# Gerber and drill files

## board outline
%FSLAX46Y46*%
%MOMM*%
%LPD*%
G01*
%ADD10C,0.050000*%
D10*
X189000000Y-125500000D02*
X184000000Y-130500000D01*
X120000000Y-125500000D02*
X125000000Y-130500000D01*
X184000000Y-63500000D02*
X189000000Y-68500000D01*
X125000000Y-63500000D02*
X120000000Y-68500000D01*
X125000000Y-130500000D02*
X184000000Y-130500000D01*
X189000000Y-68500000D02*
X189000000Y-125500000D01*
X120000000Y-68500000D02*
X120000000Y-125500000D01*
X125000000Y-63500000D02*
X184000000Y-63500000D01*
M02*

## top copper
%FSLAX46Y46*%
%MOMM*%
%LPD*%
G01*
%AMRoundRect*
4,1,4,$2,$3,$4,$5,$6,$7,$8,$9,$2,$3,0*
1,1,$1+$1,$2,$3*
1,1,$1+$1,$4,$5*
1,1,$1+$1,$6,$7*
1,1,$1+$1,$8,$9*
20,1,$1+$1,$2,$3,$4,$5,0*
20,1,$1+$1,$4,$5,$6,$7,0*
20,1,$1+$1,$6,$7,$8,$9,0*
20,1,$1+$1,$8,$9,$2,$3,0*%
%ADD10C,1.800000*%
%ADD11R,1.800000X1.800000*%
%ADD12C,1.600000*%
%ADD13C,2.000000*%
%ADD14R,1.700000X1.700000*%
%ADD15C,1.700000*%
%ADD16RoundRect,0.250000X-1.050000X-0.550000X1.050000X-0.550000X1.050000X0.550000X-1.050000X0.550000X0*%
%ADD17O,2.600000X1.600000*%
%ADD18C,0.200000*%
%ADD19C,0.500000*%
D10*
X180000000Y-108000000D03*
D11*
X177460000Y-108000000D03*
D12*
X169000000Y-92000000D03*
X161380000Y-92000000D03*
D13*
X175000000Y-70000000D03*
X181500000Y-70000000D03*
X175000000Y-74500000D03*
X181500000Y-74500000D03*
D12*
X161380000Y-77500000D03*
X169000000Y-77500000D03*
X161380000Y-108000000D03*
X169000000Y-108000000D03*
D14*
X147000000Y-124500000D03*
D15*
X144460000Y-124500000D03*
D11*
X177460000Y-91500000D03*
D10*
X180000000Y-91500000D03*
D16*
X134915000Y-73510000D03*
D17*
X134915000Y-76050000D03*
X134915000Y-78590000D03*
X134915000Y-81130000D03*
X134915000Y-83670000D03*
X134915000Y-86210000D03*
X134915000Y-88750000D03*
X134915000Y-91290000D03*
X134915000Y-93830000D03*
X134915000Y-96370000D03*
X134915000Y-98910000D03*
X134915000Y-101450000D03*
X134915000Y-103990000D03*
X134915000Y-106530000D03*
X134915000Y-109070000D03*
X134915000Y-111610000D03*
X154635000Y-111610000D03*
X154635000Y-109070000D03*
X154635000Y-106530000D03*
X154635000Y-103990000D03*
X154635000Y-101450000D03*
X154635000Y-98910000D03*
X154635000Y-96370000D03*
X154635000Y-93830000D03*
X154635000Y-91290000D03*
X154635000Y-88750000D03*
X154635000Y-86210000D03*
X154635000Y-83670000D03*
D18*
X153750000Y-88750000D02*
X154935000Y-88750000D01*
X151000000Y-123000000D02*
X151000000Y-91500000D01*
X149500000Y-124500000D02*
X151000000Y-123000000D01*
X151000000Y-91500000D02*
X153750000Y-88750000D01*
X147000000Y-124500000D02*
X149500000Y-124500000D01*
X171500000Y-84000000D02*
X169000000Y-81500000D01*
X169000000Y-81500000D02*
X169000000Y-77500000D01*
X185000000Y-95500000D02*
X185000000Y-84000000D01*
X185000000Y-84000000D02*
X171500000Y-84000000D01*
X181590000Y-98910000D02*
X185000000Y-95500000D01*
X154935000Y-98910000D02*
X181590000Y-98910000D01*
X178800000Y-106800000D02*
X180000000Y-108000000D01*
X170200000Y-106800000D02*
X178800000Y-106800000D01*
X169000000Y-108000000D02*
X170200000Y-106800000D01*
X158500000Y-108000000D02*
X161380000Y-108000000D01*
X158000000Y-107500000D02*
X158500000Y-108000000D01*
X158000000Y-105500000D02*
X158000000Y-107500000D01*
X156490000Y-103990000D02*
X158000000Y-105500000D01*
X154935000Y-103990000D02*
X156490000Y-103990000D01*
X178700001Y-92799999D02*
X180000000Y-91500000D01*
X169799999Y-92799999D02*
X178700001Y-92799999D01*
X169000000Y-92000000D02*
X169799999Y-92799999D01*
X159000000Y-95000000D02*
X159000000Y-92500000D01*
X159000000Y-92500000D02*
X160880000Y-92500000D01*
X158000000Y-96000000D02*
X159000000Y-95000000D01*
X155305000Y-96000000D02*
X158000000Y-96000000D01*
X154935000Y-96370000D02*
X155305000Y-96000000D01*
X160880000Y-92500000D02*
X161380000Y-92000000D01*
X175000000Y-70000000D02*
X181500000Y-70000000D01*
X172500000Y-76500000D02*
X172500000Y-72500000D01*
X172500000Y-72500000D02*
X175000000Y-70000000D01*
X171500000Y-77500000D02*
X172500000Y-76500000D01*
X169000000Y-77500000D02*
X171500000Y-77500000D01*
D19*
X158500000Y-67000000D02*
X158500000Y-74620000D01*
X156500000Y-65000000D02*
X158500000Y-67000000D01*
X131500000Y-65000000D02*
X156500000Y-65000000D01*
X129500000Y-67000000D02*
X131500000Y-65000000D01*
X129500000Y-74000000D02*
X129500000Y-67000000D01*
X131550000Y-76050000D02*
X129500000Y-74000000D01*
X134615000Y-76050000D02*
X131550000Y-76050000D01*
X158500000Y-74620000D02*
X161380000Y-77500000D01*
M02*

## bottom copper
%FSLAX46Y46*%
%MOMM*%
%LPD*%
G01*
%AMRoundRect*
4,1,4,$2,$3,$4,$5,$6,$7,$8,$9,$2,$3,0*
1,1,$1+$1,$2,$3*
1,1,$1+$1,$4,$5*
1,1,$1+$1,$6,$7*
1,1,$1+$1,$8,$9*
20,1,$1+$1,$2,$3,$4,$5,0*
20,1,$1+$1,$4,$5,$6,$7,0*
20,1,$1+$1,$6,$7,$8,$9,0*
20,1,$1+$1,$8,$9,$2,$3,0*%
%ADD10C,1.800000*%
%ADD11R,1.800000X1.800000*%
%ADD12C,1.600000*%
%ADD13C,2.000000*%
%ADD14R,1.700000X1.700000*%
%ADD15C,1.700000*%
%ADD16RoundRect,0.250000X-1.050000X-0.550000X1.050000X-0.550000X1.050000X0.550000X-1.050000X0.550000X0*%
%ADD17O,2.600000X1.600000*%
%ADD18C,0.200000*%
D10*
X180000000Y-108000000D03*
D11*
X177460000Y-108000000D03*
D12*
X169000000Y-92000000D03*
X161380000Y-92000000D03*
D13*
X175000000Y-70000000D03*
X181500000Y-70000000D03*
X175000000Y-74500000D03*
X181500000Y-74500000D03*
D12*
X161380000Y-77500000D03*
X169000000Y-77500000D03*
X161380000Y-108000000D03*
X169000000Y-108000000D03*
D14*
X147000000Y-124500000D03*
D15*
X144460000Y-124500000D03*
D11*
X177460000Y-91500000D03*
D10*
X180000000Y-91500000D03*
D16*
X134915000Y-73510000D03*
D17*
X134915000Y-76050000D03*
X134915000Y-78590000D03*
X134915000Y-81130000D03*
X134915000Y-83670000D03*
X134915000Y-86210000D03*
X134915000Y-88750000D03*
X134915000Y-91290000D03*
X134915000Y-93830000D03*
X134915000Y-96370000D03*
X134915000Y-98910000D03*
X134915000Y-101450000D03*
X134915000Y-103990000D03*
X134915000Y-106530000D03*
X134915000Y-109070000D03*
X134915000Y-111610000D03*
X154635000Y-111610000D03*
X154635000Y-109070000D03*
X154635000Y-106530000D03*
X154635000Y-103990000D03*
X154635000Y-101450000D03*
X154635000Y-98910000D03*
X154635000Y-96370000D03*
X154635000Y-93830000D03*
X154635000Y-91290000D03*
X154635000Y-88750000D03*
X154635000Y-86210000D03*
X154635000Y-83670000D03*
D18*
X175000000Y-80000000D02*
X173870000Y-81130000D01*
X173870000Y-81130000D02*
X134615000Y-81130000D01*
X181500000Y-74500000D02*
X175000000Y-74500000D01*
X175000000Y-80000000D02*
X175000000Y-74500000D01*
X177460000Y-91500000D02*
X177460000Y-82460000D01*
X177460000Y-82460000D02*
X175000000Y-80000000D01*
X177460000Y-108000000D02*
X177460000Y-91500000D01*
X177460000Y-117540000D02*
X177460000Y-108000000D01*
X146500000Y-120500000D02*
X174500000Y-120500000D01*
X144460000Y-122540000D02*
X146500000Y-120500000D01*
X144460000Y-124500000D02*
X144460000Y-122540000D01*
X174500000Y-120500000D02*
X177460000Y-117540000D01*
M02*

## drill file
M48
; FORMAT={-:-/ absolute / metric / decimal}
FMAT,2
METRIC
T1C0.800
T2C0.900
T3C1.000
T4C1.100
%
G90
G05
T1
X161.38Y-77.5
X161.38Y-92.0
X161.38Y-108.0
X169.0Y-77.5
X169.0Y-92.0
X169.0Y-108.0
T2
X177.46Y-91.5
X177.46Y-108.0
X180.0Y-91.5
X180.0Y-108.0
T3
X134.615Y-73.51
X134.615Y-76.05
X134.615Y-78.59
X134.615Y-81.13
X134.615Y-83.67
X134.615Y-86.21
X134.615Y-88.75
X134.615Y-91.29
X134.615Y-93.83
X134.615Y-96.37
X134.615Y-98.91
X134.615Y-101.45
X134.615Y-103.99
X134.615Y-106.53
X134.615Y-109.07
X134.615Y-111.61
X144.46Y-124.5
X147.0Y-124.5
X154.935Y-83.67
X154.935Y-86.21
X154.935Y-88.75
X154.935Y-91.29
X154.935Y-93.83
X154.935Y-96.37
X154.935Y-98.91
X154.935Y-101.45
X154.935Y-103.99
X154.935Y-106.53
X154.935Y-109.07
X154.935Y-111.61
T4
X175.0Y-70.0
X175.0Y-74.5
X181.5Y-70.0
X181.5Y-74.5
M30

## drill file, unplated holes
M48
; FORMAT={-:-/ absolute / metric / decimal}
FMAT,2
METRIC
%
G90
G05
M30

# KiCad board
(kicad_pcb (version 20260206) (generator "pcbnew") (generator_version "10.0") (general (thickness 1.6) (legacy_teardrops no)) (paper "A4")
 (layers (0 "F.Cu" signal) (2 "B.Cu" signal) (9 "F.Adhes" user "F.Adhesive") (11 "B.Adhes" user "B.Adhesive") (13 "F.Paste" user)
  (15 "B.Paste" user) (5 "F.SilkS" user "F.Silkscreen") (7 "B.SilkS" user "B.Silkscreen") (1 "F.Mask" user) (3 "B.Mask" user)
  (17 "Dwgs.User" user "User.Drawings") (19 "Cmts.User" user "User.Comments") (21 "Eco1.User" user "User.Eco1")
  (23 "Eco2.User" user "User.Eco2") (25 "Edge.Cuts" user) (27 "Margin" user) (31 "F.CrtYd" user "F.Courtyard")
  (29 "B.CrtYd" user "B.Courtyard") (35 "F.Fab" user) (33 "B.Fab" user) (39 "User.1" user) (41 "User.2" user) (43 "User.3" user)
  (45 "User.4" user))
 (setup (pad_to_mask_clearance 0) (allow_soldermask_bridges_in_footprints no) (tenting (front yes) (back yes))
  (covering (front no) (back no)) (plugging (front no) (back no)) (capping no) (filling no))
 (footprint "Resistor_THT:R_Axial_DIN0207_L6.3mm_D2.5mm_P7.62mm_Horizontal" (layer "F.Cu") (at 161.38 108)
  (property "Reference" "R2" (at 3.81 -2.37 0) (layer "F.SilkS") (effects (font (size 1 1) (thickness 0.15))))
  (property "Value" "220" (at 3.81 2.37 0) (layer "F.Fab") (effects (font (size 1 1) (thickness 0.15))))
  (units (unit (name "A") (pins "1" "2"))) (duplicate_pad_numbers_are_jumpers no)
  (pad "1" thru_hole circle (at 0 0) (size 1.6 1.6) (drill 0.8) (layers "*.Cu" "*.Mask") (remove_unused_layers no)
   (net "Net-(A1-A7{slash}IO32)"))
  (pad "2" thru_hole circle (at 7.62 0) (size 1.6 1.6) (drill 0.8) (layers "*.Cu" "*.Mask") (remove_unused_layers no) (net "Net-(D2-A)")))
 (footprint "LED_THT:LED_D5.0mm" (layer "F.Cu") (at 177.46 91.5)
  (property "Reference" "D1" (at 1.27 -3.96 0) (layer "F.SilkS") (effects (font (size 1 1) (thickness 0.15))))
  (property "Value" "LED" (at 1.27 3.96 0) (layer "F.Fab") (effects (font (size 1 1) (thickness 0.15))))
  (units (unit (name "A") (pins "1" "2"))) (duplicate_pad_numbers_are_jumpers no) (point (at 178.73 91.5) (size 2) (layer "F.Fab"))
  (pad "1" thru_hole rect (at 0 0) (size 1.8 1.8) (drill 0.9) (layers "*.Cu" "*.Mask") (remove_unused_layers no) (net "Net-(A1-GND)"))
  (pad "2" thru_hole circle (at 2.54 0) (size 1.8 1.8) (drill 0.9) (layers "*.Cu" "*.Mask") (remove_unused_layers no) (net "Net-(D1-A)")))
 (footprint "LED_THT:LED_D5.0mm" (layer "F.Cu") (at 177.46 108)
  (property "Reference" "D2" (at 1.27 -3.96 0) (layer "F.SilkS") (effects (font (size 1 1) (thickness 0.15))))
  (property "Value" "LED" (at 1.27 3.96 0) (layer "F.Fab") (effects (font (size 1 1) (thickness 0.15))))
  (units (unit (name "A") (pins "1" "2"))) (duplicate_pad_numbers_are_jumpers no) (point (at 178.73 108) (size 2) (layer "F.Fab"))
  (pad "1" thru_hole rect (at 0 0) (size 1.8 1.8) (drill 0.9) (layers "*.Cu" "*.Mask") (remove_unused_layers no) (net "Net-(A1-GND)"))
  (pad "2" thru_hole circle (at 2.54 0) (size 1.8 1.8) (drill 0.9) (layers "*.Cu" "*.Mask") (remove_unused_layers no) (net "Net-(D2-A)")))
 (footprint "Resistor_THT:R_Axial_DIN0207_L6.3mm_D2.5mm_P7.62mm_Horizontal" (layer "F.Cu") (at 161.38 92)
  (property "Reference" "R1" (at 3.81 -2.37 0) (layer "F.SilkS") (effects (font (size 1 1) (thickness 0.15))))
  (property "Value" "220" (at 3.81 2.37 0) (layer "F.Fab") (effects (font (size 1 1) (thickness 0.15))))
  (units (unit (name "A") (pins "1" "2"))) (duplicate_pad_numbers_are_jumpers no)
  (pad "1" thru_hole circle (at 0 0) (size 1.6 1.6) (drill 0.8) (layers "*.Cu" "*.Mask") (remove_unused_layers no)
   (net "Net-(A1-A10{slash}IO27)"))
  (pad "2" thru_hole circle (at 7.62 0) (size 1.6 1.6) (drill 0.8) (layers "*.Cu" "*.Mask") (remove_unused_layers no) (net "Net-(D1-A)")))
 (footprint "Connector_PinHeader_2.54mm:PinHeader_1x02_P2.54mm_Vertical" (layer "F.Cu") (at 147 124.5 -90)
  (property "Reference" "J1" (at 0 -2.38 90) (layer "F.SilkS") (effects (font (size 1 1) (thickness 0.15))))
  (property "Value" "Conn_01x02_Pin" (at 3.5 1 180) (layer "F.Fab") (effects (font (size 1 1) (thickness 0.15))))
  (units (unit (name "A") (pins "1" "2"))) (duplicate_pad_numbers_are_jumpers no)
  (pad "1" thru_hole rect (at 0 0 270) (size 1.7 1.7) (drill 1) (layers "*.Cu" "*.Mask") (remove_unused_layers no) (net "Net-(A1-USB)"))
  (pad "2" thru_hole circle (at 0 2.54 270) (size 1.7 1.7) (drill 1) (layers "*.Cu" "*.Mask") (remove_unused_layers no) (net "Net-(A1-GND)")))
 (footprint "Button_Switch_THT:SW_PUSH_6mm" (layer "F.Cu") (at 175 70)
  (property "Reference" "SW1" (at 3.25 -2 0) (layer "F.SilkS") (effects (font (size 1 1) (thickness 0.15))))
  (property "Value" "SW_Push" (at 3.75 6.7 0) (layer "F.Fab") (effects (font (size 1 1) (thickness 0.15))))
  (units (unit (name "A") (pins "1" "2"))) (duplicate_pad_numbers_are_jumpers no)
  (pad "1" thru_hole circle (at 0 0 90) (size 2 2) (drill 1.1) (layers "*.Cu" "*.Mask") (remove_unused_layers no)
   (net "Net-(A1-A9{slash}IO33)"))
  (pad "1" thru_hole circle (at 6.5 0 90) (size 2 2) (drill 1.1) (layers "*.Cu" "*.Mask") (remove_unused_layers no)
   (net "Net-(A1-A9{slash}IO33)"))
  (pad "2" thru_hole circle (at 0 4.5 90) (size 2 2) (drill 1.1) (layers "*.Cu" "*.Mask") (remove_unused_layers no) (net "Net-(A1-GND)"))
  (pad "2" thru_hole circle (at 6.5 4.5 90) (size 2 2) (drill 1.1) (layers "*.Cu" "*.Mask") (remove_unused_layers no) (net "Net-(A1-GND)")))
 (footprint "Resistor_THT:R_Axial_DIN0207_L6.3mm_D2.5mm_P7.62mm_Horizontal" (layer "F.Cu") (at 161.38 77.5)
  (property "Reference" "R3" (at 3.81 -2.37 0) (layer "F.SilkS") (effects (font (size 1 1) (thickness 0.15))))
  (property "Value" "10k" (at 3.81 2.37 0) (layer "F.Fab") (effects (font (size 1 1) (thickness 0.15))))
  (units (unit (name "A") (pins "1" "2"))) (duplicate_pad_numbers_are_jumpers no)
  (pad "1" thru_hole circle (at 0 0) (size 1.6 1.6) (drill 0.8) (layers "*.Cu" "*.Mask") (remove_unused_layers no) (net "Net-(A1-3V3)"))
  (pad "2" thru_hole circle (at 7.62 0) (size 1.6 1.6) (drill 0.8) (layers "*.Cu" "*.Mask") (remove_unused_layers no)
   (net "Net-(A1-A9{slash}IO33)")))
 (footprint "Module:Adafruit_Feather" (layer "F.Cu") (at 134.615 73.51)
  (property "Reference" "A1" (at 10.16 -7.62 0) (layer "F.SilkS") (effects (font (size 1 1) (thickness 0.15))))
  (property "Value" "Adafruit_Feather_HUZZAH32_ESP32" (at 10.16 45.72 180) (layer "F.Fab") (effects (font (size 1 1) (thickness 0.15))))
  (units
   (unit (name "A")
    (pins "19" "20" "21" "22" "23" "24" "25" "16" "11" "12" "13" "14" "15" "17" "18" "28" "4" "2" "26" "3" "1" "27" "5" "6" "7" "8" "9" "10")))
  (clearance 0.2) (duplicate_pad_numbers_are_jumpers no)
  (pad "1" thru_hole roundrect (at 0 0) (size 2.6 1.6) (drill 1 (offset 0.3 0)) (layers "*.Cu" "*.Mask") (remove_unused_layers no)
   (roundrect_rratio 0.15625) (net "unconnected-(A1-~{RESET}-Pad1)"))
  (pad "2" thru_hole oval (at 0 2.54) (size 2.6 1.6) (drill 1 (offset 0.3 0)) (layers "*.Cu" "*.Mask") (remove_unused_layers no)
   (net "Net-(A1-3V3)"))
  (pad "3" thru_hole oval (at 0 5.08) (size 2.6 1.6) (drill 1 (offset 0.3 0)) (layers "*.Cu" "*.Mask") (remove_unused_layers no)
   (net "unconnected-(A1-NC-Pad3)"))
  (pad "4" thru_hole oval (at 0 7.62) (size 2.6 1.6) (drill 1 (offset 0.3 0)) (layers "*.Cu" "*.Mask") (remove_unused_layers no)
   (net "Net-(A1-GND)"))
  (pad "5" thru_hole oval (at 0 10.16) (size 2.6 1.6) (drill 1 (offset 0.3 0)) (layers "*.Cu" "*.Mask") (remove_unused_layers no)
   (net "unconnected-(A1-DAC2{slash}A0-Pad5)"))
  (pad "6" thru_hole oval (at 0 12.7) (size 2.6 1.6) (drill 1 (offset 0.3 0)) (layers "*.Cu" "*.Mask") (remove_unused_layers no)
   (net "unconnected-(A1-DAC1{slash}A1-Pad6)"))
  (pad "7" thru_hole oval (at 0 15.24) (size 2.6 1.6) (drill 1 (offset 0.3 0)) (layers "*.Cu" "*.Mask") (remove_unused_layers no)
   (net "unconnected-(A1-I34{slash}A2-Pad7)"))
  (pad "8" thru_hole oval (at 0 17.78) (size 2.6 1.6) (drill 1 (offset 0.3 0)) (layers "*.Cu" "*.Mask") (remove_unused_layers no)
   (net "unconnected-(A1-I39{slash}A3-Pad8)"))
  (pad "9" thru_hole oval (at 0 20.32) (size 2.6 1.6) (drill 1 (offset 0.3 0)) (layers "*.Cu" "*.Mask") (remove_unused_layers no)
   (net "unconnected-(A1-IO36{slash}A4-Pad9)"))
  (pad "10" thru_hole oval (at 0 22.86) (size 2.6 1.6) (drill 1 (offset 0.3 0)) (layers "*.Cu" "*.Mask") (remove_unused_layers no)
   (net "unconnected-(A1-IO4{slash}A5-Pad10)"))
  (pad "11" thru_hole oval (at 0 25.4) (size 2.6 1.6) (drill 1 (offset 0.3 0)) (layers "*.Cu" "*.Mask") (remove_unused_layers no)
   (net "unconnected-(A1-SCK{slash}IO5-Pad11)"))
  (pad "12" thru_hole oval (at 0 27.94) (size 2.6 1.6) (drill 1 (offset 0.3 0)) (layers "*.Cu" "*.Mask") (remove_unused_layers no)
   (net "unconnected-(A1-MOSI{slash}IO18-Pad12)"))
  (pad "13" thru_hole oval (at 0 30.48) (size 2.6 1.6) (drill 1 (offset 0.3 0)) (layers "*.Cu" "*.Mask") (remove_unused_layers no)
   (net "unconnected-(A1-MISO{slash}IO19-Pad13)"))
  (pad "14" thru_hole oval (at 0 33.02) (size 2.6 1.6) (drill 1 (offset 0.3 0)) (layers "*.Cu" "*.Mask") (remove_unused_layers no)
   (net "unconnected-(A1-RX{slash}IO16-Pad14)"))
  (pad "15" thru_hole oval (at 0 35.56) (size 2.6 1.6) (drill 1 (offset 0.3 0)) (layers "*.Cu" "*.Mask") (remove_unused_layers no)
   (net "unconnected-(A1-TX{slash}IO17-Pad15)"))
  (pad "16" thru_hole oval (at 0 38.1) (size 2.6 1.6) (drill 1 (offset 0.3 0)) (layers "*.Cu" "*.Mask") (remove_unused_layers no)
   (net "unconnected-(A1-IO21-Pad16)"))
  (pad "17" thru_hole oval (at 20.32 38.1 180) (size 2.6 1.6) (drill 1 (offset 0.3 0)) (layers "*.Cu" "*.Mask") (remove_unused_layers no)
   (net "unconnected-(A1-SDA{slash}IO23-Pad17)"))
  (pad "18" thru_hole oval (at 20.32 35.56 180) (size 2.6 1.6) (drill 1 (offset 0.3 0)) (layers "*.Cu" "*.Mask") (remove_unused_layers no)
   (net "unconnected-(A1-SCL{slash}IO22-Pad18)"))
  (pad "19" thru_hole oval (at 20.32 33.02 180) (size 2.6 1.6) (drill 1 (offset 0.3 0)) (layers "*.Cu" "*.Mask") (remove_unused_layers no)
   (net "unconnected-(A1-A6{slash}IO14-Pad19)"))
  (pad "20" thru_hole oval (at 20.32 30.48 180) (size 2.6 1.6) (drill 1 (offset 0.3 0)) (layers "*.Cu" "*.Mask") (remove_unused_layers no)
   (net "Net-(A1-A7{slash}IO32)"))
  (pad "21" thru_hole oval (at 20.32 27.94 180) (size 2.6 1.6) (drill 1 (offset 0.3 0)) (layers "*.Cu" "*.Mask") (remove_unused_layers no)
   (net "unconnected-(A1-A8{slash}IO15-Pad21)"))
  (pad "22" thru_hole oval (at 20.32 25.4 180) (size 2.6 1.6) (drill 1 (offset 0.3 0)) (layers "*.Cu" "*.Mask") (remove_unused_layers no)
   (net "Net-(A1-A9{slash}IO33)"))
  (pad "23" thru_hole oval (at 20.32 22.86 180) (size 2.6 1.6) (drill 1 (offset 0.3 0)) (layers "*.Cu" "*.Mask") (remove_unused_layers no)
   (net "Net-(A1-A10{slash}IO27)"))
  (pad "24" thru_hole oval (at 20.32 20.32 180) (size 2.6 1.6) (drill 1 (offset 0.3 0)) (layers "*.Cu" "*.Mask") (remove_unused_layers no)
   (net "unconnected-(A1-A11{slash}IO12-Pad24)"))
  (pad "25" thru_hole oval (at 20.32 17.78 180) (size 2.6 1.6) (drill 1 (offset 0.3 0)) (layers "*.Cu" "*.Mask") (remove_unused_layers no)
   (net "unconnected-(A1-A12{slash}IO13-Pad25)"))
  (pad "26" thru_hole oval (at 20.32 15.24 180) (size 2.6 1.6) (drill 1 (offset 0.3 0)) (layers "*.Cu" "*.Mask") (remove_unused_layers no)
   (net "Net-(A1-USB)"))
  (pad "27" thru_hole oval (at 20.32 12.7 180) (size 2.6 1.6) (drill 1 (offset 0.3 0)) (layers "*.Cu" "*.Mask") (remove_unused_layers no)
   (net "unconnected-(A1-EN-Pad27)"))
  (pad "28" thru_hole oval (at 20.32 10.16 180) (size 2.6 1.6) (drill 1 (offset 0.3 0)) (layers "*.Cu" "*.Mask") (remove_unused_layers no)
   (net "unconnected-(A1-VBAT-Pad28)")))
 (gr_line (start 120 68.5) (end 120 125.5) (stroke (width 0.05) (type default)) (layer "Edge.Cuts"))
 (gr_line (start 120 125.5) (end 125 130.5) (stroke (width 0.05) (type default)) (layer "Edge.Cuts"))
 (gr_line (start 125 63.5) (end 120 68.5) (stroke (width 0.05) (type default)) (layer "Edge.Cuts"))
 (gr_line (start 125 63.5) (end 184 63.5) (stroke (width 0.05) (type default)) (layer "Edge.Cuts"))
 (gr_line (start 125 130.5) (end 184 130.5) (stroke (width 0.05) (type default)) (layer "Edge.Cuts"))
 (gr_line (start 184 63.5) (end 189 68.5) (stroke (width 0.05) (type default)) (layer "Edge.Cuts"))
 (gr_line (start 189 68.5) (end 189 125.5) (stroke (width 0.05) (type default)) (layer "Edge.Cuts"))
 (gr_line (start 189 125.5) (end 184 130.5) (stroke (width 0.05) (type default)) (layer "Edge.Cuts"))
 (segment (start 154.935 96.37) (end 155.305 96) (width 0.2) (layer "F.Cu") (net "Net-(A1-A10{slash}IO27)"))
 (segment (start 159 95) (end 159 92.5) (width 0.2) (layer "F.Cu") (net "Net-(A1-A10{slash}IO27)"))
 (segment (start 155.305 96) (end 158 96) (width 0.2) (layer "F.Cu") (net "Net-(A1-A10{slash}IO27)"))
 (segment (start 159 92.5) (end 160.88 92.5) (width 0.2) (layer "F.Cu") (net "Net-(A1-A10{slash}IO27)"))
 (segment (start 160.88 92.5) (end 161.38 92) (width 0.2) (layer "F.Cu") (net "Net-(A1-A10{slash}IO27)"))
 (segment (start 158 96) (end 159 95) (width 0.2) (layer "F.Cu") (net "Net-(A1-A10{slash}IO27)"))
 (segment (start 172.5 72.5) (end 175 70) (width 0.2) (layer "F.Cu") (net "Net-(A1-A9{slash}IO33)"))
 (segment (start 154.935 98.91) (end 181.59 98.91) (width 0.2) (layer "F.Cu") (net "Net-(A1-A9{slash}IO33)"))
 (segment (start 181.59 98.91) (end 185 95.5) (width 0.2) (layer "F.Cu") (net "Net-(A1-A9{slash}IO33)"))
 (segment (start 171.5 84) (end 169 81.5) (width 0.2) (layer "F.Cu") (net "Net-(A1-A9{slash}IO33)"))
 (segment (start 175 70) (end 181.5 70) (width 0.2) (layer "F.Cu") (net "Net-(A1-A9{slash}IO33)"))
 (segment (start 172.5 76.5) (end 172.5 72.5) (width 0.2) (layer "F.Cu") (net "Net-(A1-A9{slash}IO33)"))
 (segment (start 171.5 77.5) (end 172.5 76.5) (width 0.2) (layer "F.Cu") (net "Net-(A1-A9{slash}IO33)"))
 (segment (start 185 95.5) (end 185 84) (width 0.2) (layer "F.Cu") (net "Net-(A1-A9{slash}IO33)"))
 (segment (start 169 77.5) (end 171.5 77.5) (width 0.2) (layer "F.Cu") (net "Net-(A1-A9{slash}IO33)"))
 (segment (start 169 81.5) (end 169 77.5) (width 0.2) (layer "F.Cu") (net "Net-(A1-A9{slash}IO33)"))
 (segment (start 185 84) (end 171.5 84) (width 0.2) (layer "F.Cu") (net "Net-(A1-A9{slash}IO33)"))
 (segment (start 154.935 103.99) (end 156.49 103.99) (width 0.2) (layer "F.Cu") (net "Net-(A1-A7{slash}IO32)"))
 (segment (start 158 107.5) (end 158.5 108) (width 0.2) (layer "F.Cu") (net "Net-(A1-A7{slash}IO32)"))
 (segment (start 158 105.5) (end 158 107.5) (width 0.2) (layer "F.Cu") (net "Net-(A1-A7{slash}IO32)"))
 (segment (start 158.5 108) (end 161.38 108) (width 0.2) (layer "F.Cu") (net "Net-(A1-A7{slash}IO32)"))
 (segment (start 156.49 103.99) (end 158 105.5) (width 0.2) (layer "F.Cu") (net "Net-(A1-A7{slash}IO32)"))
 (segment (start 146.5 120.5) (end 174.5 120.5) (width 0.2) (layer "B.Cu") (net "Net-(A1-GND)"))
 (segment (start 173.87 81.13) (end 134.615 81.13) (width 0.2) (layer "B.Cu") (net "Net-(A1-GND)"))
 (segment (start 177.46 82.46) (end 175 80) (width 0.2) (layer "B.Cu") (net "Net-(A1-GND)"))
 (segment (start 177.46 91.5) (end 177.46 82.46) (width 0.2) (layer "B.Cu") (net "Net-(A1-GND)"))
 (segment (start 144.46 124.5) (end 144.46 122.54) (width 0.2) (layer "B.Cu") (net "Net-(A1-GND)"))
 (segment (start 177.46 117.54) (end 177.46 108) (width 0.2) (layer "B.Cu") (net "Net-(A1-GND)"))
 (segment (start 175 80) (end 175 74.5) (width 0.2) (layer "B.Cu") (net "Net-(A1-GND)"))
 (segment (start 177.46 108) (end 177.46 91.5) (width 0.2) (layer "B.Cu") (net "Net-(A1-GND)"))
 (segment (start 174.5 120.5) (end 177.46 117.54) (width 0.2) (layer "B.Cu") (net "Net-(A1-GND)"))
 (segment (start 144.46 122.54) (end 146.5 120.5) (width 0.2) (layer "B.Cu") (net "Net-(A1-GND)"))
 (segment (start 181.5 74.5) (end 175 74.5) (width 0.2) (layer "B.Cu") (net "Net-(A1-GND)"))
 (segment (start 175 80) (end 173.87 81.13) (width 0.2) (layer "B.Cu") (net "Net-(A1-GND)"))
 (segment (start 149.5 124.5) (end 151 123) (width 0.2) (layer "F.Cu") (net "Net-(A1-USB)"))
 (segment (start 151 123) (end 151 91.5) (width 0.2) (layer "F.Cu") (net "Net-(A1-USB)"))
 (segment (start 151 91.5) (end 153.75 88.75) (width 0.2) (layer "F.Cu") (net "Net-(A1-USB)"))
 (segment (start 153.75 88.75) (end 154.935 88.75) (width 0.2) (layer "F.Cu") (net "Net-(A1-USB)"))
 (segment (start 147 124.5) (end 149.5 124.5) (width 0.2) (layer "F.Cu") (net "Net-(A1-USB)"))
 (segment (start 131.55 76.05) (end 129.5 74) (width 0.5) (layer "F.Cu") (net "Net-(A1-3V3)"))
 (segment (start 129.5 67) (end 131.5 65) (width 0.5) (layer "F.Cu") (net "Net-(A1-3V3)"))
 (segment (start 134.615 76.05) (end 131.55 76.05) (width 0.5) (layer "F.Cu") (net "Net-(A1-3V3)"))
 (segment (start 158.5 67) (end 158.5 74.62) (width 0.5) (layer "F.Cu") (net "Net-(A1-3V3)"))
 (segment (start 156.5 65) (end 158.5 67) (width 0.5) (layer "F.Cu") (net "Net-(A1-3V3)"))
 (segment (start 131.5 65) (end 156.5 65) (width 0.5) (layer "F.Cu") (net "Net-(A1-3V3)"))
 (segment (start 158.5 74.62) (end 161.38 77.5) (width 0.5) (layer "F.Cu") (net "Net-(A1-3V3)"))
 (segment (start 129.5 74) (end 129.5 67) (width 0.5) (layer "F.Cu") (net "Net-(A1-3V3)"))
 (segment (start 178.700001 92.799999) (end 180 91.5) (width 0.2) (layer "F.Cu") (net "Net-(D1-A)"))
 (segment (start 169.799999 92.799999) (end 178.700001 92.799999) (width 0.2) (layer "F.Cu") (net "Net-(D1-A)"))
 (segment (start 169 92) (end 169.799999 92.799999) (width 0.2) (layer "F.Cu") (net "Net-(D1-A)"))
 (segment (start 170.2 106.8) (end 178.8 106.8) (width 0.2) (layer "F.Cu") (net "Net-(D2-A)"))
 (segment (start 178.8 106.8) (end 180 108) (width 0.2) (layer "F.Cu") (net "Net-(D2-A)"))
 (segment (start 169 108) (end 170.2 106.8) (width 0.2) (layer "F.Cu") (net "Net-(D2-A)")))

